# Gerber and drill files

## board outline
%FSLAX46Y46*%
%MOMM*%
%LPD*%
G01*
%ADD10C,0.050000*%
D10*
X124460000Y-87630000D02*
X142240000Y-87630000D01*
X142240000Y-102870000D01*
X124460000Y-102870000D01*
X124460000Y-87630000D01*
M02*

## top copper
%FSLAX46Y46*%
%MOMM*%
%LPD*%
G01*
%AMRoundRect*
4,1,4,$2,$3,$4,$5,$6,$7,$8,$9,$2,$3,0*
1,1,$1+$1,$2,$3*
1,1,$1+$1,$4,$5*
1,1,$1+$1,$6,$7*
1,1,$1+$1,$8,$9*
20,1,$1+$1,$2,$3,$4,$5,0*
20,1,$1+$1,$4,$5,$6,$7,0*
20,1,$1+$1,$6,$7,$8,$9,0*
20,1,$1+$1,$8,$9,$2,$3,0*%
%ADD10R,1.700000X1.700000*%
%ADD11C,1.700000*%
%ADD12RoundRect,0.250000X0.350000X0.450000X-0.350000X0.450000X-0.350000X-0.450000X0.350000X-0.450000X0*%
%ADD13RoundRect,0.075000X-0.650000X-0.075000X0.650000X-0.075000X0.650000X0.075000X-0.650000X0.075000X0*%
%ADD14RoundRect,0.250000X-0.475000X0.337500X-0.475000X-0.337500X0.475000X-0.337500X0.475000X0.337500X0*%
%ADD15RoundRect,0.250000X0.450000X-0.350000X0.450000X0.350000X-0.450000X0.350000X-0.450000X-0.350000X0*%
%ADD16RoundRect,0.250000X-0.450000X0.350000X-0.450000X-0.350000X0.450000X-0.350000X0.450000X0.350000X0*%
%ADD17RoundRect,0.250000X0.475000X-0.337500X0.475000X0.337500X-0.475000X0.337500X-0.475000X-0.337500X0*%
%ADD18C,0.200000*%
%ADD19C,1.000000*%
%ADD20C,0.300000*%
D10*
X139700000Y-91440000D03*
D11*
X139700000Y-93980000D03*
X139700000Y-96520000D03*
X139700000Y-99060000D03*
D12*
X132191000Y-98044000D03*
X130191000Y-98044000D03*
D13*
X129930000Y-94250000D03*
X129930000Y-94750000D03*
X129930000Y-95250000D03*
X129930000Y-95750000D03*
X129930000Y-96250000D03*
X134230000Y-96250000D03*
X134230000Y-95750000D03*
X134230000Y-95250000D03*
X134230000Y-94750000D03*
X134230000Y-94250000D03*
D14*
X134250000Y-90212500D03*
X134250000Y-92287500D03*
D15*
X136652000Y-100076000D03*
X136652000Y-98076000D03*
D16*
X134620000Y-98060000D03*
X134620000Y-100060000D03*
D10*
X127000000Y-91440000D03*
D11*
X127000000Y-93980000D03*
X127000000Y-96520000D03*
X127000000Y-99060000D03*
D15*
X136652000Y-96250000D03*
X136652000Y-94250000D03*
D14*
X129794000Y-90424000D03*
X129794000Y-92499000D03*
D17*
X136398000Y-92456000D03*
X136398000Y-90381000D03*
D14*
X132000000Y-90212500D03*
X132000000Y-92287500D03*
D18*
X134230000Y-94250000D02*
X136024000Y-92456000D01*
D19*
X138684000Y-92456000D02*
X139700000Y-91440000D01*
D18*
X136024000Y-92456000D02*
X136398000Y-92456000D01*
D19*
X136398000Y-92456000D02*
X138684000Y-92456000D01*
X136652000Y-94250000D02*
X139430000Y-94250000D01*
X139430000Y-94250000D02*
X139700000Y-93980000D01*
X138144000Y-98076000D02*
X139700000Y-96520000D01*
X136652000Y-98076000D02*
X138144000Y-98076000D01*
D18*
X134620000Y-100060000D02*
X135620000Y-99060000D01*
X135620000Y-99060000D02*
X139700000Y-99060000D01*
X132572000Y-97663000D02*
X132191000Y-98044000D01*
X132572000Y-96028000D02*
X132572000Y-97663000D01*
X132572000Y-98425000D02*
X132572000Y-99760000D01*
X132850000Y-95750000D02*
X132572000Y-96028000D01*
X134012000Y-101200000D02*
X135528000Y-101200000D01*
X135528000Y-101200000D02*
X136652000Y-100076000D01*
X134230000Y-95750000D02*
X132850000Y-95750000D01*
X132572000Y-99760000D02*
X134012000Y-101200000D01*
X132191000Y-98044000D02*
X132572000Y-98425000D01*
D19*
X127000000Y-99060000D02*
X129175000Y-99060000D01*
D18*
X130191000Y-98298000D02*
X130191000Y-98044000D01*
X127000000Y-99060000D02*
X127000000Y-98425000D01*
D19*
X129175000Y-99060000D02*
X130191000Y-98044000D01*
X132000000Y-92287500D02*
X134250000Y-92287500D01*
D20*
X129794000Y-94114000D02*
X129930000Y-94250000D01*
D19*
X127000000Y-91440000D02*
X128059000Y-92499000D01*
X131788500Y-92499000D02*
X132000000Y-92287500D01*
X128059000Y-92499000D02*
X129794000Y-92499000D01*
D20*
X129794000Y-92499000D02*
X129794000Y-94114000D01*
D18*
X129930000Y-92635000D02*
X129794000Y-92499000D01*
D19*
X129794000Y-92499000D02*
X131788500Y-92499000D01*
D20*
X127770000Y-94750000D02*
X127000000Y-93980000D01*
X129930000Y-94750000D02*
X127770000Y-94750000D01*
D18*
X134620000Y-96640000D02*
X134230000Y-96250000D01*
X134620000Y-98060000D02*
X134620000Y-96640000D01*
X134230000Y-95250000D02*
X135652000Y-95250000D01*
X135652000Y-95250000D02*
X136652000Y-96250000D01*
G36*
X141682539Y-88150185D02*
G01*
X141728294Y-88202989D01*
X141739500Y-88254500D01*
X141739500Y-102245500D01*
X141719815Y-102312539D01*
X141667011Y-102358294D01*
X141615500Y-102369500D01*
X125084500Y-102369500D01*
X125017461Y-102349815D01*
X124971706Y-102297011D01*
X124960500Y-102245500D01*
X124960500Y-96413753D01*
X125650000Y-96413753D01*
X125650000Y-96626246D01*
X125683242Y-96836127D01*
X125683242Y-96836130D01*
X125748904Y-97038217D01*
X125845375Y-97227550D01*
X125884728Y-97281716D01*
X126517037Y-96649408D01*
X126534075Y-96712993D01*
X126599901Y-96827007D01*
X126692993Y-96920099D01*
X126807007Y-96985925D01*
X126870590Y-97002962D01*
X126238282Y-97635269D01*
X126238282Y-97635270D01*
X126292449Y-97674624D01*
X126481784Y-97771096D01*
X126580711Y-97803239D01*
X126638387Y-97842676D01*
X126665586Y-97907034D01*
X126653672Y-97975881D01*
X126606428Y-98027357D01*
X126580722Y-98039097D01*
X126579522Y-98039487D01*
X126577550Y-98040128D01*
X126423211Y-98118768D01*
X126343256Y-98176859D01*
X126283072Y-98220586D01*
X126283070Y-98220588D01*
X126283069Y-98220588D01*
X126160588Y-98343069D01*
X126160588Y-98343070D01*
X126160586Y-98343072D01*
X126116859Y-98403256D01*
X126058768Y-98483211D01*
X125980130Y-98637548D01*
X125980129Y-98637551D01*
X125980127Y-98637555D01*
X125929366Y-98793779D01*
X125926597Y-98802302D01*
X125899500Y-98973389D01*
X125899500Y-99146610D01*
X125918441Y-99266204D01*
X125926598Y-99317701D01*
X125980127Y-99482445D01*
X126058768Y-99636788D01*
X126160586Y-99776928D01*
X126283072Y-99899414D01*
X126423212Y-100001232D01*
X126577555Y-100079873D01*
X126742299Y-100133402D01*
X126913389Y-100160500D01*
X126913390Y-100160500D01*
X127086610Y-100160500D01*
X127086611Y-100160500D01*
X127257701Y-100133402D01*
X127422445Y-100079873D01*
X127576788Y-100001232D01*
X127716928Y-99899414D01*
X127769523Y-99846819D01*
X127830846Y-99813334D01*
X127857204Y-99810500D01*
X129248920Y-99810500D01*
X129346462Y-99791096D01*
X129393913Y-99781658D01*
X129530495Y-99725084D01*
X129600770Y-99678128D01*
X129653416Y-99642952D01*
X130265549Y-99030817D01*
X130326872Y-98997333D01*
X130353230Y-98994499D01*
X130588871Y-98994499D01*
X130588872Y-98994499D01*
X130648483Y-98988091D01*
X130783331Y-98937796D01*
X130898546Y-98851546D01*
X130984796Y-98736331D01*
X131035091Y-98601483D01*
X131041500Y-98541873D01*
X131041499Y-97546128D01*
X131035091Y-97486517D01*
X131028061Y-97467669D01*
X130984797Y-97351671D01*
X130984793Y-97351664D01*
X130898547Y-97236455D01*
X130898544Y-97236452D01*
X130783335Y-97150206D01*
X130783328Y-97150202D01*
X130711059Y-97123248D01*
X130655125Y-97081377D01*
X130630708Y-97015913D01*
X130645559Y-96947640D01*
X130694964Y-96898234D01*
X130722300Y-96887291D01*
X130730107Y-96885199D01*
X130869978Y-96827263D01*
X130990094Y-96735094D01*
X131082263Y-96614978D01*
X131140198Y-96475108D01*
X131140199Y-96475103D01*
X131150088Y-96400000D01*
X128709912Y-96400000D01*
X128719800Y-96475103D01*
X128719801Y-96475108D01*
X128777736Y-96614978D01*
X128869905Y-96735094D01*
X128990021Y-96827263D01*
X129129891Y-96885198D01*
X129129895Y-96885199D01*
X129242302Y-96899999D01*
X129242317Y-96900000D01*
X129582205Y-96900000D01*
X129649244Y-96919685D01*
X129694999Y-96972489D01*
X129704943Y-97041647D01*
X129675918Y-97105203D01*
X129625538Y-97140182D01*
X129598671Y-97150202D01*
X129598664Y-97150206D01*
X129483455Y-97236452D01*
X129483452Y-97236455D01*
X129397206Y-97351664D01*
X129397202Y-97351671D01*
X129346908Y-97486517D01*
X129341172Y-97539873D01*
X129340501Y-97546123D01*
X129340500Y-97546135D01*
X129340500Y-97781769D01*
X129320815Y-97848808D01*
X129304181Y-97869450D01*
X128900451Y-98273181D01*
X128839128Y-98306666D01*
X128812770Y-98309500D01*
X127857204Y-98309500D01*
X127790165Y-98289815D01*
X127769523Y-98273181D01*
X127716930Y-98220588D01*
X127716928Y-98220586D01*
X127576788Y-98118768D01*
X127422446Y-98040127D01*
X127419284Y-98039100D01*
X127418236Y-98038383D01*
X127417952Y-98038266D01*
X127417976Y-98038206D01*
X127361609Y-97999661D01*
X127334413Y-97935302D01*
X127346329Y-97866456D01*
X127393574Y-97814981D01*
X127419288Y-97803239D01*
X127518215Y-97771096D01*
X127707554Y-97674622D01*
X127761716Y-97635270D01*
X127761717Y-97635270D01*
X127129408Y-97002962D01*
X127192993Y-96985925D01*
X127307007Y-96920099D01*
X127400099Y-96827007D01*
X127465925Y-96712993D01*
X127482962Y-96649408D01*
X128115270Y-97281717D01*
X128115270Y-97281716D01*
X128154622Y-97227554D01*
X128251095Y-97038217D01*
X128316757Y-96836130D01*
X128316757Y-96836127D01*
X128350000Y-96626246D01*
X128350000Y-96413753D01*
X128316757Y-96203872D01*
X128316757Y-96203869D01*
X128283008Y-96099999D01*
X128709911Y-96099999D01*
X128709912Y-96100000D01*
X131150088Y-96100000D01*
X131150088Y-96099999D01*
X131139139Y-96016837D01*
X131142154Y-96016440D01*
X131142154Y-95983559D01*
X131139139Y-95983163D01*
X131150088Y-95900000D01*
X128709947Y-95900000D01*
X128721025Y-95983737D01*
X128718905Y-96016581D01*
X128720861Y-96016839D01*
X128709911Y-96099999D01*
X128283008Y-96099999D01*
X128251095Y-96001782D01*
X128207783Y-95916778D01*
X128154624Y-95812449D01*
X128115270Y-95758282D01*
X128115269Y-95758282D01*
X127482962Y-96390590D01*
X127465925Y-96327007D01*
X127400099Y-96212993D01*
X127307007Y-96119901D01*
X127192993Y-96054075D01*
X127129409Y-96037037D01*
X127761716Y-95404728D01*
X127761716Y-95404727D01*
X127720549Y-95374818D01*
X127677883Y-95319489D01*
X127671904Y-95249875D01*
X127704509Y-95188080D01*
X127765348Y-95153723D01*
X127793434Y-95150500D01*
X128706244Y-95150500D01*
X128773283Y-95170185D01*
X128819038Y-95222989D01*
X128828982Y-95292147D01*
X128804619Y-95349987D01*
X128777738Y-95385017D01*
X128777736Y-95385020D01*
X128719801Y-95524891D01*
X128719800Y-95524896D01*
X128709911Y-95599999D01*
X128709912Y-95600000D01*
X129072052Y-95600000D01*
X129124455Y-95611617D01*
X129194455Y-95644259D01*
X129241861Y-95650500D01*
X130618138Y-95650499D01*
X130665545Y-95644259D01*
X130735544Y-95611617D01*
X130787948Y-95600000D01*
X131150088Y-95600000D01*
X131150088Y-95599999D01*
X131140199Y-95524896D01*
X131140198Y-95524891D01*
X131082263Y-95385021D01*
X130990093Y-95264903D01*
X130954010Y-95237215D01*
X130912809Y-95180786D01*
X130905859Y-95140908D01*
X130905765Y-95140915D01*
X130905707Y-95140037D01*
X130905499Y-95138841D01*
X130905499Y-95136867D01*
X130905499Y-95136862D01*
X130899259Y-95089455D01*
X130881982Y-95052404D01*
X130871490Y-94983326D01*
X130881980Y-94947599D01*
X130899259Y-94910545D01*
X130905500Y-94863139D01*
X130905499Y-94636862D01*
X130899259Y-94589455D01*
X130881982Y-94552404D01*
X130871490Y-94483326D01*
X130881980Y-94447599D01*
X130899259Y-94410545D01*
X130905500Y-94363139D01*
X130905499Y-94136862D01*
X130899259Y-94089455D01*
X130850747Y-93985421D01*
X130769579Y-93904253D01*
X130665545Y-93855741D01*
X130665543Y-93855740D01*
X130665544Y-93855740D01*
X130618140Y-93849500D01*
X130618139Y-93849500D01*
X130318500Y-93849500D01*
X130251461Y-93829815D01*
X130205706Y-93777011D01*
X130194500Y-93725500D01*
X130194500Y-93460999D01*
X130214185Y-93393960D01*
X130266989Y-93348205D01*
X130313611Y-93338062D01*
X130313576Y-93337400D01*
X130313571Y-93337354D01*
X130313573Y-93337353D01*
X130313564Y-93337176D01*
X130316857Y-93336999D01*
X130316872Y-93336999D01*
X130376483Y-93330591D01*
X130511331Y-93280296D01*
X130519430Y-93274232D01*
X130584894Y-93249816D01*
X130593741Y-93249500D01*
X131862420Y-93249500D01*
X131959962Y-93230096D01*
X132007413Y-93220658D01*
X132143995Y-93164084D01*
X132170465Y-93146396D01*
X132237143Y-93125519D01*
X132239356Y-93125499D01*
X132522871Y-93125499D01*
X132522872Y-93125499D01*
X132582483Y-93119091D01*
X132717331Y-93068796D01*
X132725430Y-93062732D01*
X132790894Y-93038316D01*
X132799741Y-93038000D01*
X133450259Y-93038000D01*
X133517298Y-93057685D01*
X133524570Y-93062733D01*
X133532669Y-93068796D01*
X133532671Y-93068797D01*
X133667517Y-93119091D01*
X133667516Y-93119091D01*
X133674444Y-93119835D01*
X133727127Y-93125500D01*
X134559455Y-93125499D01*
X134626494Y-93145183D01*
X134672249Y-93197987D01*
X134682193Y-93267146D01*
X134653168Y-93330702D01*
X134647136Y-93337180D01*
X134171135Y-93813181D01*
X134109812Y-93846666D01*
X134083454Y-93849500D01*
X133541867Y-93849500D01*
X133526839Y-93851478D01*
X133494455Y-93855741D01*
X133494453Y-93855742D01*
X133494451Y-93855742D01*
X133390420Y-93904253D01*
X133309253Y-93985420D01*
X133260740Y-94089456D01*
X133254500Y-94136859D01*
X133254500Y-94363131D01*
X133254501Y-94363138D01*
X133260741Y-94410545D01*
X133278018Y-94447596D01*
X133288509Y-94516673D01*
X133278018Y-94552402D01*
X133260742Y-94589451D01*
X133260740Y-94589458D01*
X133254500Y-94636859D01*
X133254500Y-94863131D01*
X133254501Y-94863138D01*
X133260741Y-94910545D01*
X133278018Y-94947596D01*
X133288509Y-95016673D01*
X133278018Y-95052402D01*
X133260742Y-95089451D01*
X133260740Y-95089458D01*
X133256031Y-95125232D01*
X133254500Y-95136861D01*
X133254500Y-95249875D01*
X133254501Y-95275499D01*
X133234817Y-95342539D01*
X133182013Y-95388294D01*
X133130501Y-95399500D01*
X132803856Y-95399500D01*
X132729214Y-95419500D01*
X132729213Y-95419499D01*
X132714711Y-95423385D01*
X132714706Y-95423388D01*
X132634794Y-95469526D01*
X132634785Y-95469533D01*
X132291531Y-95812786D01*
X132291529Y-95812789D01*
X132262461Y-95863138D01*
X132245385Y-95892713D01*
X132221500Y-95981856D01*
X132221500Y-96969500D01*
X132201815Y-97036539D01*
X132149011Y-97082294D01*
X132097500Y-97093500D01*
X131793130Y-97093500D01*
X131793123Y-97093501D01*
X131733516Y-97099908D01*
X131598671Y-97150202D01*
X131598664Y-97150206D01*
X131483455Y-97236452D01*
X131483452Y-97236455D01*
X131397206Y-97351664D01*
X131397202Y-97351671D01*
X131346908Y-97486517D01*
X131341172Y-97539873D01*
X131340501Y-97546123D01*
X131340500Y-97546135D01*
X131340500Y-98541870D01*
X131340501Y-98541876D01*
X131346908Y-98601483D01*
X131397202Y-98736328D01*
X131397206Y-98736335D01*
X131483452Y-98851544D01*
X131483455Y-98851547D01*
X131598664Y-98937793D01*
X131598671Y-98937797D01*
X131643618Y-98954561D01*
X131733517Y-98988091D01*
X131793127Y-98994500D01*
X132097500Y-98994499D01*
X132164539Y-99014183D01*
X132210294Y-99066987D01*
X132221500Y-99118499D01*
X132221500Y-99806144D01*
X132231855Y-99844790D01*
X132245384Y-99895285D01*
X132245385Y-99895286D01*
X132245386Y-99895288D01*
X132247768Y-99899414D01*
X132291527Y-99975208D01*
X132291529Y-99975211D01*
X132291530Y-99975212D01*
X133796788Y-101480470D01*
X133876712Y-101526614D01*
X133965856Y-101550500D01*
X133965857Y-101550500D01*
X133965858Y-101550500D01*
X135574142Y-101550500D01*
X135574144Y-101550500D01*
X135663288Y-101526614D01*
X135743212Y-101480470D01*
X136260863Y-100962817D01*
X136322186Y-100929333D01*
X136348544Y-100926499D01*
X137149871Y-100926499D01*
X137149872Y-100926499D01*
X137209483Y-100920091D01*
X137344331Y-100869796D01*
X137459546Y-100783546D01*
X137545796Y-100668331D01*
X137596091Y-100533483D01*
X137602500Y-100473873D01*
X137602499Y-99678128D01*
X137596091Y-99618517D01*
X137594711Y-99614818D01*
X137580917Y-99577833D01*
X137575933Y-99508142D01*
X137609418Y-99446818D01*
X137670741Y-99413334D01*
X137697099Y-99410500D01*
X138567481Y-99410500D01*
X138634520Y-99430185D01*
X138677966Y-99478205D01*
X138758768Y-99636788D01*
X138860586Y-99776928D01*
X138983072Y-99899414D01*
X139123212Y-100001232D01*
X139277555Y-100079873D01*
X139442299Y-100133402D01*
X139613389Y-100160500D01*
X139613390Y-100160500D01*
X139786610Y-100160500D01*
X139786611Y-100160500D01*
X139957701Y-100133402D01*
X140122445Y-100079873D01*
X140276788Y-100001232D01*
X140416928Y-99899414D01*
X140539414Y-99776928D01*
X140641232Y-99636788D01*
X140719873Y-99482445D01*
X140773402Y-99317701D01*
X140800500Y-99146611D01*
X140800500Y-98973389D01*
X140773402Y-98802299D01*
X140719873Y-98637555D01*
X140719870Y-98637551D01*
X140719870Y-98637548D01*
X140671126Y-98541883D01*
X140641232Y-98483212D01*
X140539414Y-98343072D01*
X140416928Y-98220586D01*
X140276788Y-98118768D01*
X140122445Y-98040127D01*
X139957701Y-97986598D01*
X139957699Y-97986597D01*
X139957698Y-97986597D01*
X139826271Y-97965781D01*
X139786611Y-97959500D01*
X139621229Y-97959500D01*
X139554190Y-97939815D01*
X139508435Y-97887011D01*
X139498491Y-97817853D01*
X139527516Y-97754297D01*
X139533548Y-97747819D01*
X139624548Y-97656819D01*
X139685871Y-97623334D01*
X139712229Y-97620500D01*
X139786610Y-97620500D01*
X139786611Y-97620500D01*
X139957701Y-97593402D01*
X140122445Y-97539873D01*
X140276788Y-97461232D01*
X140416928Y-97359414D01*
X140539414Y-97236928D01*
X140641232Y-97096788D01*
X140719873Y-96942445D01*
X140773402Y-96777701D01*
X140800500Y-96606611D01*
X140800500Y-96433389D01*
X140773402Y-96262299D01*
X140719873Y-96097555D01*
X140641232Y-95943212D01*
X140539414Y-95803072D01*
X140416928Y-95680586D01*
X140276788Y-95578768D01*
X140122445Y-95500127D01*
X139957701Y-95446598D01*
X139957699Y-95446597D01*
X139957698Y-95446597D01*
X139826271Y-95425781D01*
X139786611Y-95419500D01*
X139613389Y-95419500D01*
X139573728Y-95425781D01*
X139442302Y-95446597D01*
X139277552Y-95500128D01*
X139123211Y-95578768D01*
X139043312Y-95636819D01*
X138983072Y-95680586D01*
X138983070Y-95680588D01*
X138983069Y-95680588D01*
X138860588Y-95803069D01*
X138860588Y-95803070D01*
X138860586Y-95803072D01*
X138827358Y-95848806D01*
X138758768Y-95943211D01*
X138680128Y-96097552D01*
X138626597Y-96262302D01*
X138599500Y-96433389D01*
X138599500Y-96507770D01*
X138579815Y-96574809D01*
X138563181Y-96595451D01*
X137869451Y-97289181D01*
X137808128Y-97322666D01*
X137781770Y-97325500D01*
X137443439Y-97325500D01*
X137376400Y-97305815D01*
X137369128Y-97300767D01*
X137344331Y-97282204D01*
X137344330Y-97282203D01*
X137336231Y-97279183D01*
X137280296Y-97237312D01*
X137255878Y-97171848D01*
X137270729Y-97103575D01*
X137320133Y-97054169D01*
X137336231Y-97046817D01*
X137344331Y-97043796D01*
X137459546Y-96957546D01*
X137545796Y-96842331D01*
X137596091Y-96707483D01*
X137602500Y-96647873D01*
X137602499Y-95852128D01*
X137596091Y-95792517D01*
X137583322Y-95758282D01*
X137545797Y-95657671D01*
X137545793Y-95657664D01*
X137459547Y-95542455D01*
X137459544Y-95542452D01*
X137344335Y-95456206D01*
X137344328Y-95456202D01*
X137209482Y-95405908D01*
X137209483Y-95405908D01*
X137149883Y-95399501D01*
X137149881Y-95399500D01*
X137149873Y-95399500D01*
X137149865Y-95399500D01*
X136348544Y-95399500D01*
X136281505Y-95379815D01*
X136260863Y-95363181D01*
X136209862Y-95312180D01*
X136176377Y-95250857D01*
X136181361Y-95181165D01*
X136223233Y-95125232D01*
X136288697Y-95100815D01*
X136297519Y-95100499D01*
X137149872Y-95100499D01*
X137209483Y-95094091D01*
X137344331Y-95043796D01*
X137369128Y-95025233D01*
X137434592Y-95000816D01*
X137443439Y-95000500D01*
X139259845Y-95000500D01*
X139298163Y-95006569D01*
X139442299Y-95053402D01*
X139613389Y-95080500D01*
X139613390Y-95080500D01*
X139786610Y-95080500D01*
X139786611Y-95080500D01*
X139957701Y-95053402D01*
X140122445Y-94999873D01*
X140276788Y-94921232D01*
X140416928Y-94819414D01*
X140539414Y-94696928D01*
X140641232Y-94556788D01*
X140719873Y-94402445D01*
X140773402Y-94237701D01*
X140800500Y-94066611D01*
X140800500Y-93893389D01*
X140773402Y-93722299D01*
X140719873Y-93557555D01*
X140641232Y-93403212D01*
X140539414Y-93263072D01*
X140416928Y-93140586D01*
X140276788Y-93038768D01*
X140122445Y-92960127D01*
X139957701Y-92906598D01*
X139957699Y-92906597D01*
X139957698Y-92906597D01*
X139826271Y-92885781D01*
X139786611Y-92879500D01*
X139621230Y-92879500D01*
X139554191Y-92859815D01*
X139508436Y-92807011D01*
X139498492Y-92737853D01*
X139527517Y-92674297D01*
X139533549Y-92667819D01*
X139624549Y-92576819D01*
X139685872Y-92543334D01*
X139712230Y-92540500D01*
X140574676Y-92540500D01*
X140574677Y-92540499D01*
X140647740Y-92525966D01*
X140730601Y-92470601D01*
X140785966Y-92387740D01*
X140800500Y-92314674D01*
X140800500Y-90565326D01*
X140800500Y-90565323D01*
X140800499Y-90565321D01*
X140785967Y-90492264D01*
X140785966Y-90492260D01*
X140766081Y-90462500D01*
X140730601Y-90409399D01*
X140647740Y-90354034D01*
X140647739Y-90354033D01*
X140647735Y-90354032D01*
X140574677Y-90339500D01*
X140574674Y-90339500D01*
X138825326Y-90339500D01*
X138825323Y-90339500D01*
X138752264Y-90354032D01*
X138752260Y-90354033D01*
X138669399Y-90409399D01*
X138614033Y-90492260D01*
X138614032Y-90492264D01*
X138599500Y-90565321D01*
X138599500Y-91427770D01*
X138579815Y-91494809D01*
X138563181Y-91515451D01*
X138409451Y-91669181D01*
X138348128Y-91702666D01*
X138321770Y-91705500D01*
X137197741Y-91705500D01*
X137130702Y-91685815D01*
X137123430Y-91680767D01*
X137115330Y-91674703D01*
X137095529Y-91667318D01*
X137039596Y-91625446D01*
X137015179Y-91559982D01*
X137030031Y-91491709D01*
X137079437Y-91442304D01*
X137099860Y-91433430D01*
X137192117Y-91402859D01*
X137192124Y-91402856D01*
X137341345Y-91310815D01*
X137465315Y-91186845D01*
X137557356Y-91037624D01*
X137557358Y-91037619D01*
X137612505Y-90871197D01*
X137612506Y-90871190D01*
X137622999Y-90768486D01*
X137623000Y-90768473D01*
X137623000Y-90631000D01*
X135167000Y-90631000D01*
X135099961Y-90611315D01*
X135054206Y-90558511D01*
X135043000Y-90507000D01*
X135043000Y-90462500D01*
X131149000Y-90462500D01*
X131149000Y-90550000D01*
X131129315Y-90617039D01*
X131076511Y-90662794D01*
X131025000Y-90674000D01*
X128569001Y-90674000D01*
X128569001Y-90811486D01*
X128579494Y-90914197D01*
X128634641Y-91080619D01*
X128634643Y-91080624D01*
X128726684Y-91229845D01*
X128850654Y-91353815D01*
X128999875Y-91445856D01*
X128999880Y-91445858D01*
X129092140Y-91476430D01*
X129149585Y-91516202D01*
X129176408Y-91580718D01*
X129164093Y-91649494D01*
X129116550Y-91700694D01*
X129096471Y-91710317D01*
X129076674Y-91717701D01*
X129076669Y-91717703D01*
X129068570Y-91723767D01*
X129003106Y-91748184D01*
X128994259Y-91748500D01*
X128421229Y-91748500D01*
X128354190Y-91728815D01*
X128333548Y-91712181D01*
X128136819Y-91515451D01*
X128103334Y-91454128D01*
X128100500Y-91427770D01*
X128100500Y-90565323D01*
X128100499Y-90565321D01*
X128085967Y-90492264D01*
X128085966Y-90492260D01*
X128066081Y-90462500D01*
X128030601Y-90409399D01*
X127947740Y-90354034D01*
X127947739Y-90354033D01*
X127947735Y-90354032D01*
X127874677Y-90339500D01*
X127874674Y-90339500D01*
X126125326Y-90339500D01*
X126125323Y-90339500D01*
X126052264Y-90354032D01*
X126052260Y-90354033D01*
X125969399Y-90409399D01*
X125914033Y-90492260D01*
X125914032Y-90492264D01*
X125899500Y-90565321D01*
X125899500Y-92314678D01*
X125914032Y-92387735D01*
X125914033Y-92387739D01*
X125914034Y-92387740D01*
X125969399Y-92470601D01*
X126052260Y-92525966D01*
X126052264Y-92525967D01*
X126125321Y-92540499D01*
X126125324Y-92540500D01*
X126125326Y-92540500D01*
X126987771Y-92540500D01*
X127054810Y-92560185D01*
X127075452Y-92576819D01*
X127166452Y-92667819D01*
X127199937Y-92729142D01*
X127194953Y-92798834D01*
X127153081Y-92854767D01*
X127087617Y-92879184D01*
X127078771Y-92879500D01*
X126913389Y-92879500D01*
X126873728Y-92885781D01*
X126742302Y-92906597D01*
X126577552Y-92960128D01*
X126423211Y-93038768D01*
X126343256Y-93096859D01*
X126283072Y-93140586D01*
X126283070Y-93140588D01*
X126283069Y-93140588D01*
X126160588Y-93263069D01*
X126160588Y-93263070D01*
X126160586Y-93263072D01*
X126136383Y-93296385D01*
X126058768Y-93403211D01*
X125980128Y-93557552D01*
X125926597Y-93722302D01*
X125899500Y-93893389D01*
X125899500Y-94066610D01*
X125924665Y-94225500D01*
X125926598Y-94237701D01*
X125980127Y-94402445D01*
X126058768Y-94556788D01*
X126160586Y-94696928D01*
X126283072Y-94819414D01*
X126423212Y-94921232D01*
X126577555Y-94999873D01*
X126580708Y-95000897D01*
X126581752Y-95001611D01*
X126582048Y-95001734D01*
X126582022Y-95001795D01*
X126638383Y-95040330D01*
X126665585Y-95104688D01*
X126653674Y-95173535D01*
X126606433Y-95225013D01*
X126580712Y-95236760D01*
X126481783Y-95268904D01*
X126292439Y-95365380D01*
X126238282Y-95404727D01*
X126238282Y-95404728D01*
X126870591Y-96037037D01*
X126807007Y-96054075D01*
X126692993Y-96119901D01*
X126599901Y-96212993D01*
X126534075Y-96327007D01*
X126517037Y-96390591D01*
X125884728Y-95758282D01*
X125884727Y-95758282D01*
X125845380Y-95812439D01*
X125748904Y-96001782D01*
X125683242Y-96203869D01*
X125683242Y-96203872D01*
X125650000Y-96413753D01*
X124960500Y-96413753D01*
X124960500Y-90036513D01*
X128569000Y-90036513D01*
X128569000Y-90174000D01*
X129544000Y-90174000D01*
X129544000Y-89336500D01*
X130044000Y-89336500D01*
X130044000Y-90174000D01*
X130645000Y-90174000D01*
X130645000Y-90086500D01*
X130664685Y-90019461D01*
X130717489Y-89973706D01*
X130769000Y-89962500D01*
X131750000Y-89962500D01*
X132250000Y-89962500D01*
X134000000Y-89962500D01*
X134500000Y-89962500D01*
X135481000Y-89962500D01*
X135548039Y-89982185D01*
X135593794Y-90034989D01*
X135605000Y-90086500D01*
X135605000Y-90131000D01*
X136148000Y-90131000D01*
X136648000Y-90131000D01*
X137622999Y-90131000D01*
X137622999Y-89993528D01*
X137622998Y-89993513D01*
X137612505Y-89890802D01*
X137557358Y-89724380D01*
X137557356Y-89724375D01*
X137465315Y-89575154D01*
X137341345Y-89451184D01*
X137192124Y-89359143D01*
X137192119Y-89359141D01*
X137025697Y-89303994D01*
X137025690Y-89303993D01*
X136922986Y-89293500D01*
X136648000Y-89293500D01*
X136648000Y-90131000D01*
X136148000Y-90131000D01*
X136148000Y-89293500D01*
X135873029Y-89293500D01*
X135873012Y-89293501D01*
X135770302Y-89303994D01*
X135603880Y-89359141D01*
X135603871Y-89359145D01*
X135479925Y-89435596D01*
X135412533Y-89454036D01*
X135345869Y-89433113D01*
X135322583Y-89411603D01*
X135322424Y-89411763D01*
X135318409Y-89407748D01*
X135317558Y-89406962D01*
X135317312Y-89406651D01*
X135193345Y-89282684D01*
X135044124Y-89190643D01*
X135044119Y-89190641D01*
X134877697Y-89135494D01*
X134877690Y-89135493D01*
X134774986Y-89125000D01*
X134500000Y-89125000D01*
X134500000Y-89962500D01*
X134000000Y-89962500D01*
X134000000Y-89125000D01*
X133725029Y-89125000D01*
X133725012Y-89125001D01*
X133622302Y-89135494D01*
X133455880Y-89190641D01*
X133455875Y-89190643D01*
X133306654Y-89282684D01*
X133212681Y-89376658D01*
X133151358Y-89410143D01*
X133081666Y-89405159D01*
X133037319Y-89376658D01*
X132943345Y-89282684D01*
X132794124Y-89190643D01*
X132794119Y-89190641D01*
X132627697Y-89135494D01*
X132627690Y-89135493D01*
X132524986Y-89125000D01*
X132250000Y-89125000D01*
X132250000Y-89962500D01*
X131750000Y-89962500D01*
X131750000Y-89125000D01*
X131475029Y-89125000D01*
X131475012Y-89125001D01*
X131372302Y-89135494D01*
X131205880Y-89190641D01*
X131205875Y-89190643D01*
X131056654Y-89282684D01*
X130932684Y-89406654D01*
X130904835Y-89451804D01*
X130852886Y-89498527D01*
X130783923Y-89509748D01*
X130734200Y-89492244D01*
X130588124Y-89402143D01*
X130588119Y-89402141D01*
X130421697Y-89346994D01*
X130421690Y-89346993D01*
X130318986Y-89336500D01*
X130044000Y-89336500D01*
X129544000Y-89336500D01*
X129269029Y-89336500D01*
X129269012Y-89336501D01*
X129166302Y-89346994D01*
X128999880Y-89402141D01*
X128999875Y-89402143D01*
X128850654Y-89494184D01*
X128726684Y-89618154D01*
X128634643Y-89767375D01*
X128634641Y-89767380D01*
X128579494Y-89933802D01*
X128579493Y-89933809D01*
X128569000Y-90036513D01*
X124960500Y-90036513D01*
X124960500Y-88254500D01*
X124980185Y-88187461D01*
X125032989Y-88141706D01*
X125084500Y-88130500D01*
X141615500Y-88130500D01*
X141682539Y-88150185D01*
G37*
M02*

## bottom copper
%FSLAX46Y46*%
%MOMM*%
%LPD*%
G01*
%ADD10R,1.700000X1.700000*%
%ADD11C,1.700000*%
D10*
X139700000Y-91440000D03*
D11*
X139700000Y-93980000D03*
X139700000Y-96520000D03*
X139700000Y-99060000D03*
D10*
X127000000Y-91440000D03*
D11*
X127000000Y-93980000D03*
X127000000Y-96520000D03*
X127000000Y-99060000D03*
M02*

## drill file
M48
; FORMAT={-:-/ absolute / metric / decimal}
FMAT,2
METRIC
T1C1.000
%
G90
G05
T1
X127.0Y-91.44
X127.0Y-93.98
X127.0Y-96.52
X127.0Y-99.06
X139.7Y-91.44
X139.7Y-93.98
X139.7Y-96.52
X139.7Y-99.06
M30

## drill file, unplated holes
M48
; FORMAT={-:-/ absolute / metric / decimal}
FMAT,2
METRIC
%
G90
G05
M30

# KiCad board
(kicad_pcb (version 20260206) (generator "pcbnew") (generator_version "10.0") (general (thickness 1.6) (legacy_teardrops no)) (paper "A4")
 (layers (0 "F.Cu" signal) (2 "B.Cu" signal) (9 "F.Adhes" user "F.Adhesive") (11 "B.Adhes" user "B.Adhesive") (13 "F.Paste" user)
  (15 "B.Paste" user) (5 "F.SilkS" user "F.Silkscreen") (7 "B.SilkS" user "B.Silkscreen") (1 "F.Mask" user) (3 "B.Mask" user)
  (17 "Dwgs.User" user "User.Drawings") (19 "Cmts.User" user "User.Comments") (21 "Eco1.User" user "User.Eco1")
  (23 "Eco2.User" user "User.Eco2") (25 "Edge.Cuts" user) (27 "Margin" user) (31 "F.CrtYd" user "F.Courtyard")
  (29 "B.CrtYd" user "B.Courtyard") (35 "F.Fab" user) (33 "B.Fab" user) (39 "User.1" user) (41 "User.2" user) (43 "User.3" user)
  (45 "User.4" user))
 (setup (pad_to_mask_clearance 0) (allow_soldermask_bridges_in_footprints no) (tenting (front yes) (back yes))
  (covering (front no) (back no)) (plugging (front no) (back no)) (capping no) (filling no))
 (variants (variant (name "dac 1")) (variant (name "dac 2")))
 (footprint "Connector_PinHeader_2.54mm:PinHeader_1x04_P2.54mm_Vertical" (layer "F.Cu") (at 139.7 91.44)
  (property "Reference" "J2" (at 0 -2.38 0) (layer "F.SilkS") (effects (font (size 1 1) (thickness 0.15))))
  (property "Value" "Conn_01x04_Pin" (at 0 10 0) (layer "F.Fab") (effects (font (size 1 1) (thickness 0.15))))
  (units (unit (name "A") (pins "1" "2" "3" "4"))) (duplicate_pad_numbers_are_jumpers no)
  (pad "1" thru_hole rect (at 0 0) (size 1.7 1.7) (drill 1) (layers "*.Cu" "*.Mask") (remove_unused_layers no) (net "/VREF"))
  (pad "2" thru_hole circle (at 0 2.54) (size 1.7 1.7) (drill 1) (layers "*.Cu" "*.Mask") (remove_unused_layers no) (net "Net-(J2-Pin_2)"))
  (pad "3" thru_hole circle (at 0 5.08) (size 1.7 1.7) (drill 1) (layers "*.Cu" "*.Mask") (remove_unused_layers no) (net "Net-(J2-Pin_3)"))
  (pad "4" thru_hole circle (at 0 7.62) (size 1.7 1.7) (drill 1) (layers "*.Cu" "*.Mask") (remove_unused_layers no) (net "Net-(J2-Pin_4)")))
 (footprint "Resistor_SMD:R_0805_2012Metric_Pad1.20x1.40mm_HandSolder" (layer "F.Cu") (at 131.191 98.044 180)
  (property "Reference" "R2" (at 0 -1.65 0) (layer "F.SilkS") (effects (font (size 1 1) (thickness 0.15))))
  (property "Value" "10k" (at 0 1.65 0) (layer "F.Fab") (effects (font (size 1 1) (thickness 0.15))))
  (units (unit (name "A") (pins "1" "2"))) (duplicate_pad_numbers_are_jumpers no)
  (pad "1" smd roundrect (at -1 0 180) (size 1.2 1.4) (layers "F.Cu" "F.Mask" "F.Paste") (roundrect_rratio 0.208333) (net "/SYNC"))
  (pad "2" smd roundrect (at 1 0 180) (size 1.2 1.4) (layers "F.Cu" "F.Mask" "F.Paste") (roundrect_rratio 0.208333) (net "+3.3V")))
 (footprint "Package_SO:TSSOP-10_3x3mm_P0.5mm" (layer "F.Cu") (at 132.08 95.25)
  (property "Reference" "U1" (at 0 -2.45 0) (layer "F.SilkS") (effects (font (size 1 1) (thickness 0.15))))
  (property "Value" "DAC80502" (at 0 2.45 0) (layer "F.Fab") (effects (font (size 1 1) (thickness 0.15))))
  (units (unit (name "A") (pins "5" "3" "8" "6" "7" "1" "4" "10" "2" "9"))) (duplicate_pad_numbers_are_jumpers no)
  (pad "1" smd roundrect (at -2.15 -1) (size 1.45 0.3) (layers "F.Cu" "F.Mask" "F.Paste") (roundrect_rratio 0.25) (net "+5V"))
  (pad "2" smd roundrect (at -2.15 -0.5) (size 1.45 0.3) (layers "F.Cu" "F.Mask" "F.Paste") (roundrect_rratio 0.25) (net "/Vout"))
  (pad "3" smd roundrect (at -2.15 0) (size 1.45 0.3) (layers "F.Cu" "F.Mask" "F.Paste") (roundrect_rratio 0.25)
   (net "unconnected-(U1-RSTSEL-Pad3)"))
  (pad "4" smd roundrect (at -2.15 0.5) (size 1.45 0.3) (layers "F.Cu" "F.Mask" "F.Paste") (roundrect_rratio 0.25) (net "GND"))
  (pad "5" smd roundrect (at -2.15 1) (size 1.45 0.3) (layers "F.Cu" "F.Mask" "F.Paste") (roundrect_rratio 0.25) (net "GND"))
  (pad "6" smd roundrect (at 2.15 1) (size 1.45 0.3) (layers "F.Cu" "F.Mask" "F.Paste") (roundrect_rratio 0.25) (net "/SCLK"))
  (pad "7" smd roundrect (at 2.15 0.5) (size 1.45 0.3) (layers "F.Cu" "F.Mask" "F.Paste") (roundrect_rratio 0.25) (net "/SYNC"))
  (pad "8" smd roundrect (at 2.15 0) (size 1.45 0.3) (layers "F.Cu" "F.Mask" "F.Paste") (roundrect_rratio 0.25) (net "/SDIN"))
  (pad "9" smd roundrect (at 2.15 -0.5) (size 1.45 0.3) (layers "F.Cu" "F.Mask" "F.Paste") (roundrect_rratio 0.25)
   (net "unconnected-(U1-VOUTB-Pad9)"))
  (pad "10" smd roundrect (at 2.15 -1) (size 1.45 0.3) (layers "F.Cu" "F.Mask" "F.Paste") (roundrect_rratio 0.25) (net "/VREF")))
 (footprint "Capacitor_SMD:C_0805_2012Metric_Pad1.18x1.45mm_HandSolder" (layer "F.Cu") (at 134.25 91.25 -90)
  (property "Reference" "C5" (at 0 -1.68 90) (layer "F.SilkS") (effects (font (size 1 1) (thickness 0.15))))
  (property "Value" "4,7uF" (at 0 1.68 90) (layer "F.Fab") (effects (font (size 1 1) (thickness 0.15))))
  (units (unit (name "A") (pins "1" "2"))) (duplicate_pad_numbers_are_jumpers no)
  (pad "1" smd roundrect (at -1.0375 0 270) (size 1.175 1.45) (layers "F.Cu" "F.Mask" "F.Paste") (roundrect_rratio 0.212766) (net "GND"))
  (pad "2" smd roundrect (at 1.0375 0 270) (size 1.175 1.45) (layers "F.Cu" "F.Mask" "F.Paste") (roundrect_rratio 0.212766) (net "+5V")))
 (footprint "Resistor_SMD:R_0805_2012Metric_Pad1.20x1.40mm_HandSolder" (layer "F.Cu") (at 136.652 99.076 90)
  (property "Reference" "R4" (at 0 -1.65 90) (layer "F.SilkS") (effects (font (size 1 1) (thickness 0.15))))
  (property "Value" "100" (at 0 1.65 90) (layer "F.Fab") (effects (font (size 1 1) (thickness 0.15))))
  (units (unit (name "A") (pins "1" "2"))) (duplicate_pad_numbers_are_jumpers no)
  (pad "1" smd roundrect (at -1 0 90) (size 1.2 1.4) (layers "F.Cu" "F.Mask" "F.Paste") (roundrect_rratio 0.208333) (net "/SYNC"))
  (pad "2" smd roundrect (at 1 0 90) (size 1.2 1.4) (layers "F.Cu" "F.Mask" "F.Paste") (roundrect_rratio 0.208333) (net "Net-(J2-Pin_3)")))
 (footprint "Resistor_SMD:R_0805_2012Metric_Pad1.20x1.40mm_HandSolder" (layer "F.Cu") (at 134.62 99.06 -90)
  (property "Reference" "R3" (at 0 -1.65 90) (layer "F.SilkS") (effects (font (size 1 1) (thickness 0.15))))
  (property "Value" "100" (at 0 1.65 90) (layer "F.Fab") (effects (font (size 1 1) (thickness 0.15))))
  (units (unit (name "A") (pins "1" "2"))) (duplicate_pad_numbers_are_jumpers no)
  (pad "1" smd roundrect (at -1 0 270) (size 1.2 1.4) (layers "F.Cu" "F.Mask" "F.Paste") (roundrect_rratio 0.208333) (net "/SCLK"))
  (pad "2" smd roundrect (at 1 0 270) (size 1.2 1.4) (layers "F.Cu" "F.Mask" "F.Paste") (roundrect_rratio 0.208333) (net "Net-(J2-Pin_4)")))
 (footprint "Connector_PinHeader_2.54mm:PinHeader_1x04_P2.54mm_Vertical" (layer "F.Cu") (at 127 91.44)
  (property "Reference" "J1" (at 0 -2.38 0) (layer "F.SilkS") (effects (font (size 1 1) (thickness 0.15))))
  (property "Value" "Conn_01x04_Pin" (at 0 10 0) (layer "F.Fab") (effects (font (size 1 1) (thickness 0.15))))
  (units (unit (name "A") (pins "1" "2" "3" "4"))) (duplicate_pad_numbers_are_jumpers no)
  (pad "1" thru_hole rect (at 0 0) (size 1.7 1.7) (drill 1) (layers "*.Cu" "*.Mask") (remove_unused_layers no) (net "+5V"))
  (pad "2" thru_hole circle (at 0 2.54) (size 1.7 1.7) (drill 1) (layers "*.Cu" "*.Mask") (remove_unused_layers no) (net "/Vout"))
  (pad "3" thru_hole circle (at 0 5.08) (size 1.7 1.7) (drill 1) (layers "*.Cu" "*.Mask") (remove_unused_layers no) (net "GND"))
  (pad "4" thru_hole circle (at 0 7.62) (size 1.7 1.7) (drill 1) (layers "*.Cu" "*.Mask") (remove_unused_layers no) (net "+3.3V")))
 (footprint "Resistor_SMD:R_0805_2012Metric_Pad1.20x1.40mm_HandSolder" (layer "F.Cu") (at 136.652 95.25 90)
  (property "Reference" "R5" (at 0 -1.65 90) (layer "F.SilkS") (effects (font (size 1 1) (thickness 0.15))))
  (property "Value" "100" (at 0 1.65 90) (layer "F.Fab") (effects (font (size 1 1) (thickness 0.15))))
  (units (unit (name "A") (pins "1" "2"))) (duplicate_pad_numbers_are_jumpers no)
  (pad "1" smd roundrect (at -1 0 90) (size 1.2 1.4) (layers "F.Cu" "F.Mask" "F.Paste") (roundrect_rratio 0.208333) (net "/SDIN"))
  (pad "2" smd roundrect (at 1 0 90) (size 1.2 1.4) (layers "F.Cu" "F.Mask" "F.Paste") (roundrect_rratio 0.208333) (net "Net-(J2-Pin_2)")))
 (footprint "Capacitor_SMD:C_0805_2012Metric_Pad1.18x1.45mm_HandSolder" (layer "F.Cu") (at 129.794 91.4615 -90)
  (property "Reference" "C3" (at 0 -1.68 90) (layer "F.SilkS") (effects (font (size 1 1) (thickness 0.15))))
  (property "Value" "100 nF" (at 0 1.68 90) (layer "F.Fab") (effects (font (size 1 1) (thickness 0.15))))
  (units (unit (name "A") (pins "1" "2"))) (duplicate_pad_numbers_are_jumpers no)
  (pad "1" smd roundrect (at -1.0375 0 270) (size 1.175 1.45) (layers "F.Cu" "F.Mask" "F.Paste") (roundrect_rratio 0.212766) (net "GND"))
  (pad "2" smd roundrect (at 1.0375 0 270) (size 1.175 1.45) (layers "F.Cu" "F.Mask" "F.Paste") (roundrect_rratio 0.212766) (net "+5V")))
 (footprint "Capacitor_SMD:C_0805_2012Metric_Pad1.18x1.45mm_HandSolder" (layer "F.Cu") (at 136.398 91.4185 90)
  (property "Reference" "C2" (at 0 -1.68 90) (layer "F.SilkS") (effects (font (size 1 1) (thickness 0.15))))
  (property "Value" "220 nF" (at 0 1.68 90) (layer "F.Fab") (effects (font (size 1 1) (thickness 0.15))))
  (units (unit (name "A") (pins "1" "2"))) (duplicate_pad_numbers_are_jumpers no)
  (pad "1" smd roundrect (at -1.0375 0 90) (size 1.175 1.45) (layers "F.Cu" "F.Mask" "F.Paste") (roundrect_rratio 0.212766) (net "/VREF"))
  (pad "2" smd roundrect (at 1.0375 0 90) (size 1.175 1.45) (layers "F.Cu" "F.Mask" "F.Paste") (roundrect_rratio 0.212766) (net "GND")))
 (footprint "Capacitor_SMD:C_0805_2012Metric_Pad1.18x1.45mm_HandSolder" (layer "F.Cu") (at 132 91.25 -90)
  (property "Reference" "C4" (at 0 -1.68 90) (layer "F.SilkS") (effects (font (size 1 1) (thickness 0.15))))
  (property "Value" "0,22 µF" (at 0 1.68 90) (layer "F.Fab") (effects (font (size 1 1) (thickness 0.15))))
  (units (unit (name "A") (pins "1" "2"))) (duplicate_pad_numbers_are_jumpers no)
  (pad "1" smd roundrect (at -1.0375 0 270) (size 1.175 1.45) (layers "F.Cu" "F.Mask" "F.Paste") (roundrect_rratio 0.212766) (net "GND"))
  (pad "2" smd roundrect (at 1.0375 0 270) (size 1.175 1.45) (layers "F.Cu" "F.Mask" "F.Paste") (roundrect_rratio 0.212766) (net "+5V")))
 (gr_rect (start 124.46 87.63) (end 142.24 102.87) (stroke (width 0.05) (type default)) (fill no) (layer "Edge.Cuts"))
 (segment (start 134.23 94.25) (end 136.024 92.456) (width 0.2) (layer "F.Cu") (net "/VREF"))
 (segment (start 138.684 92.456) (end 139.7 91.44) (width 1) (layer "F.Cu") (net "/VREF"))
 (segment (start 136.024 92.456) (end 136.398 92.456) (width 0.2) (layer "F.Cu") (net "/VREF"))
 (segment (start 136.398 92.456) (end 138.684 92.456) (width 1) (layer "F.Cu") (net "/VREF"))
 (segment (start 136.652 94.25) (end 139.43 94.25) (width 1) (layer "F.Cu") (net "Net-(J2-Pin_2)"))
 (segment (start 139.43 94.25) (end 139.7 93.98) (width 1) (layer "F.Cu") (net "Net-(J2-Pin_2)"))
 (segment (start 138.144 98.076) (end 139.7 96.52) (width 1) (layer "F.Cu") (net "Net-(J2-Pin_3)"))
 (segment (start 136.652 98.076) (end 138.144 98.076) (width 1) (layer "F.Cu") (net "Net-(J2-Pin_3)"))
 (segment (start 134.62 100.06) (end 135.62 99.06) (width 0.2) (layer "F.Cu") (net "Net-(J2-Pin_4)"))
 (segment (start 135.62 99.06) (end 139.7 99.06) (width 0.2) (layer "F.Cu") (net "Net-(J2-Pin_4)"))
 (segment (start 132.572 97.663) (end 132.191 98.044) (width 0.2) (layer "F.Cu") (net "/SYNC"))
 (segment (start 132.572 96.028) (end 132.572 97.663) (width 0.2) (layer "F.Cu") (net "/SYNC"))
 (segment (start 132.572 98.425) (end 132.572 99.76) (width 0.2) (layer "F.Cu") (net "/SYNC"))
 (segment (start 132.85 95.75) (end 132.572 96.028) (width 0.2) (layer "F.Cu") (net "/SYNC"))
 (segment (start 134.012 101.2) (end 135.528 101.2) (width 0.2) (layer "F.Cu") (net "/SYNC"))
 (segment (start 135.528 101.2) (end 136.652 100.076) (width 0.2) (layer "F.Cu") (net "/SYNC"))
 (segment (start 134.23 95.75) (end 132.85 95.75) (width 0.2) (layer "F.Cu") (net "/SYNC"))
 (segment (start 132.572 99.76) (end 134.012 101.2) (width 0.2) (layer "F.Cu") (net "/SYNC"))
 (segment (start 132.191 98.044) (end 132.572 98.425) (width 0.2) (layer "F.Cu") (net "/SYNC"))
 (segment (start 127 99.06) (end 129.175 99.06) (width 1) (layer "F.Cu") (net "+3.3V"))
 (segment (start 130.191 98.298) (end 130.191 98.044) (width 0.2) (layer "F.Cu") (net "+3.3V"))
 (segment (start 127 99.06) (end 127 98.425) (width 0.2) (layer "F.Cu") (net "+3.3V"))
 (segment (start 129.175 99.06) (end 130.191 98.044) (width 1) (layer "F.Cu") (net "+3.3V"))
 (segment (start 132 92.2875) (end 134.25 92.2875) (width 1) (layer "F.Cu") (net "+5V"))
 (segment (start 129.794 94.114) (end 129.93 94.25) (width 0.3) (layer "F.Cu") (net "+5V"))
 (segment (start 127 91.44) (end 128.059 92.499) (width 1) (layer "F.Cu") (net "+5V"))
 (segment (start 131.7885 92.499) (end 132 92.2875) (width 1) (layer "F.Cu") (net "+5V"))
 (segment (start 128.059 92.499) (end 129.794 92.499) (width 1) (layer "F.Cu") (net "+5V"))
 (segment (start 129.794 92.499) (end 129.794 94.114) (width 0.3) (layer "F.Cu") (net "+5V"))
 (segment (start 129.93 92.635) (end 129.794 92.499) (width 0.2) (layer "F.Cu") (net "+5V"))
 (segment (start 129.794 92.499) (end 131.7885 92.499) (width 1) (layer "F.Cu") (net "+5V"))
 (segment (start 127.77 94.75) (end 127 93.98) (width 0.3) (layer "F.Cu") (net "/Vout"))
 (segment (start 129.93 94.75) (end 127.77 94.75) (width 0.3) (layer "F.Cu") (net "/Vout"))
 (segment (start 134.62 96.64) (end 134.23 96.25) (width 0.2) (layer "F.Cu") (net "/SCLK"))
 (segment (start 134.62 98.06) (end 134.62 96.64) (width 0.2) (layer "F.Cu") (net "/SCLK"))
 (segment (start 134.23 95.25) (end 135.652 95.25) (width 0.2) (layer "F.Cu") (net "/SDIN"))
 (segment (start 135.652 95.25) (end 136.652 96.25) (width 0.2) (layer "F.Cu") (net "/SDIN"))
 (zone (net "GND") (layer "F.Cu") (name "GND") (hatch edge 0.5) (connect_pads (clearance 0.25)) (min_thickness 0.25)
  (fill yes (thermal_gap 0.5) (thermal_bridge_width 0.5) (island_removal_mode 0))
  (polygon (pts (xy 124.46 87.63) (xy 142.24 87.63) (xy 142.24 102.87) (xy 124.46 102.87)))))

